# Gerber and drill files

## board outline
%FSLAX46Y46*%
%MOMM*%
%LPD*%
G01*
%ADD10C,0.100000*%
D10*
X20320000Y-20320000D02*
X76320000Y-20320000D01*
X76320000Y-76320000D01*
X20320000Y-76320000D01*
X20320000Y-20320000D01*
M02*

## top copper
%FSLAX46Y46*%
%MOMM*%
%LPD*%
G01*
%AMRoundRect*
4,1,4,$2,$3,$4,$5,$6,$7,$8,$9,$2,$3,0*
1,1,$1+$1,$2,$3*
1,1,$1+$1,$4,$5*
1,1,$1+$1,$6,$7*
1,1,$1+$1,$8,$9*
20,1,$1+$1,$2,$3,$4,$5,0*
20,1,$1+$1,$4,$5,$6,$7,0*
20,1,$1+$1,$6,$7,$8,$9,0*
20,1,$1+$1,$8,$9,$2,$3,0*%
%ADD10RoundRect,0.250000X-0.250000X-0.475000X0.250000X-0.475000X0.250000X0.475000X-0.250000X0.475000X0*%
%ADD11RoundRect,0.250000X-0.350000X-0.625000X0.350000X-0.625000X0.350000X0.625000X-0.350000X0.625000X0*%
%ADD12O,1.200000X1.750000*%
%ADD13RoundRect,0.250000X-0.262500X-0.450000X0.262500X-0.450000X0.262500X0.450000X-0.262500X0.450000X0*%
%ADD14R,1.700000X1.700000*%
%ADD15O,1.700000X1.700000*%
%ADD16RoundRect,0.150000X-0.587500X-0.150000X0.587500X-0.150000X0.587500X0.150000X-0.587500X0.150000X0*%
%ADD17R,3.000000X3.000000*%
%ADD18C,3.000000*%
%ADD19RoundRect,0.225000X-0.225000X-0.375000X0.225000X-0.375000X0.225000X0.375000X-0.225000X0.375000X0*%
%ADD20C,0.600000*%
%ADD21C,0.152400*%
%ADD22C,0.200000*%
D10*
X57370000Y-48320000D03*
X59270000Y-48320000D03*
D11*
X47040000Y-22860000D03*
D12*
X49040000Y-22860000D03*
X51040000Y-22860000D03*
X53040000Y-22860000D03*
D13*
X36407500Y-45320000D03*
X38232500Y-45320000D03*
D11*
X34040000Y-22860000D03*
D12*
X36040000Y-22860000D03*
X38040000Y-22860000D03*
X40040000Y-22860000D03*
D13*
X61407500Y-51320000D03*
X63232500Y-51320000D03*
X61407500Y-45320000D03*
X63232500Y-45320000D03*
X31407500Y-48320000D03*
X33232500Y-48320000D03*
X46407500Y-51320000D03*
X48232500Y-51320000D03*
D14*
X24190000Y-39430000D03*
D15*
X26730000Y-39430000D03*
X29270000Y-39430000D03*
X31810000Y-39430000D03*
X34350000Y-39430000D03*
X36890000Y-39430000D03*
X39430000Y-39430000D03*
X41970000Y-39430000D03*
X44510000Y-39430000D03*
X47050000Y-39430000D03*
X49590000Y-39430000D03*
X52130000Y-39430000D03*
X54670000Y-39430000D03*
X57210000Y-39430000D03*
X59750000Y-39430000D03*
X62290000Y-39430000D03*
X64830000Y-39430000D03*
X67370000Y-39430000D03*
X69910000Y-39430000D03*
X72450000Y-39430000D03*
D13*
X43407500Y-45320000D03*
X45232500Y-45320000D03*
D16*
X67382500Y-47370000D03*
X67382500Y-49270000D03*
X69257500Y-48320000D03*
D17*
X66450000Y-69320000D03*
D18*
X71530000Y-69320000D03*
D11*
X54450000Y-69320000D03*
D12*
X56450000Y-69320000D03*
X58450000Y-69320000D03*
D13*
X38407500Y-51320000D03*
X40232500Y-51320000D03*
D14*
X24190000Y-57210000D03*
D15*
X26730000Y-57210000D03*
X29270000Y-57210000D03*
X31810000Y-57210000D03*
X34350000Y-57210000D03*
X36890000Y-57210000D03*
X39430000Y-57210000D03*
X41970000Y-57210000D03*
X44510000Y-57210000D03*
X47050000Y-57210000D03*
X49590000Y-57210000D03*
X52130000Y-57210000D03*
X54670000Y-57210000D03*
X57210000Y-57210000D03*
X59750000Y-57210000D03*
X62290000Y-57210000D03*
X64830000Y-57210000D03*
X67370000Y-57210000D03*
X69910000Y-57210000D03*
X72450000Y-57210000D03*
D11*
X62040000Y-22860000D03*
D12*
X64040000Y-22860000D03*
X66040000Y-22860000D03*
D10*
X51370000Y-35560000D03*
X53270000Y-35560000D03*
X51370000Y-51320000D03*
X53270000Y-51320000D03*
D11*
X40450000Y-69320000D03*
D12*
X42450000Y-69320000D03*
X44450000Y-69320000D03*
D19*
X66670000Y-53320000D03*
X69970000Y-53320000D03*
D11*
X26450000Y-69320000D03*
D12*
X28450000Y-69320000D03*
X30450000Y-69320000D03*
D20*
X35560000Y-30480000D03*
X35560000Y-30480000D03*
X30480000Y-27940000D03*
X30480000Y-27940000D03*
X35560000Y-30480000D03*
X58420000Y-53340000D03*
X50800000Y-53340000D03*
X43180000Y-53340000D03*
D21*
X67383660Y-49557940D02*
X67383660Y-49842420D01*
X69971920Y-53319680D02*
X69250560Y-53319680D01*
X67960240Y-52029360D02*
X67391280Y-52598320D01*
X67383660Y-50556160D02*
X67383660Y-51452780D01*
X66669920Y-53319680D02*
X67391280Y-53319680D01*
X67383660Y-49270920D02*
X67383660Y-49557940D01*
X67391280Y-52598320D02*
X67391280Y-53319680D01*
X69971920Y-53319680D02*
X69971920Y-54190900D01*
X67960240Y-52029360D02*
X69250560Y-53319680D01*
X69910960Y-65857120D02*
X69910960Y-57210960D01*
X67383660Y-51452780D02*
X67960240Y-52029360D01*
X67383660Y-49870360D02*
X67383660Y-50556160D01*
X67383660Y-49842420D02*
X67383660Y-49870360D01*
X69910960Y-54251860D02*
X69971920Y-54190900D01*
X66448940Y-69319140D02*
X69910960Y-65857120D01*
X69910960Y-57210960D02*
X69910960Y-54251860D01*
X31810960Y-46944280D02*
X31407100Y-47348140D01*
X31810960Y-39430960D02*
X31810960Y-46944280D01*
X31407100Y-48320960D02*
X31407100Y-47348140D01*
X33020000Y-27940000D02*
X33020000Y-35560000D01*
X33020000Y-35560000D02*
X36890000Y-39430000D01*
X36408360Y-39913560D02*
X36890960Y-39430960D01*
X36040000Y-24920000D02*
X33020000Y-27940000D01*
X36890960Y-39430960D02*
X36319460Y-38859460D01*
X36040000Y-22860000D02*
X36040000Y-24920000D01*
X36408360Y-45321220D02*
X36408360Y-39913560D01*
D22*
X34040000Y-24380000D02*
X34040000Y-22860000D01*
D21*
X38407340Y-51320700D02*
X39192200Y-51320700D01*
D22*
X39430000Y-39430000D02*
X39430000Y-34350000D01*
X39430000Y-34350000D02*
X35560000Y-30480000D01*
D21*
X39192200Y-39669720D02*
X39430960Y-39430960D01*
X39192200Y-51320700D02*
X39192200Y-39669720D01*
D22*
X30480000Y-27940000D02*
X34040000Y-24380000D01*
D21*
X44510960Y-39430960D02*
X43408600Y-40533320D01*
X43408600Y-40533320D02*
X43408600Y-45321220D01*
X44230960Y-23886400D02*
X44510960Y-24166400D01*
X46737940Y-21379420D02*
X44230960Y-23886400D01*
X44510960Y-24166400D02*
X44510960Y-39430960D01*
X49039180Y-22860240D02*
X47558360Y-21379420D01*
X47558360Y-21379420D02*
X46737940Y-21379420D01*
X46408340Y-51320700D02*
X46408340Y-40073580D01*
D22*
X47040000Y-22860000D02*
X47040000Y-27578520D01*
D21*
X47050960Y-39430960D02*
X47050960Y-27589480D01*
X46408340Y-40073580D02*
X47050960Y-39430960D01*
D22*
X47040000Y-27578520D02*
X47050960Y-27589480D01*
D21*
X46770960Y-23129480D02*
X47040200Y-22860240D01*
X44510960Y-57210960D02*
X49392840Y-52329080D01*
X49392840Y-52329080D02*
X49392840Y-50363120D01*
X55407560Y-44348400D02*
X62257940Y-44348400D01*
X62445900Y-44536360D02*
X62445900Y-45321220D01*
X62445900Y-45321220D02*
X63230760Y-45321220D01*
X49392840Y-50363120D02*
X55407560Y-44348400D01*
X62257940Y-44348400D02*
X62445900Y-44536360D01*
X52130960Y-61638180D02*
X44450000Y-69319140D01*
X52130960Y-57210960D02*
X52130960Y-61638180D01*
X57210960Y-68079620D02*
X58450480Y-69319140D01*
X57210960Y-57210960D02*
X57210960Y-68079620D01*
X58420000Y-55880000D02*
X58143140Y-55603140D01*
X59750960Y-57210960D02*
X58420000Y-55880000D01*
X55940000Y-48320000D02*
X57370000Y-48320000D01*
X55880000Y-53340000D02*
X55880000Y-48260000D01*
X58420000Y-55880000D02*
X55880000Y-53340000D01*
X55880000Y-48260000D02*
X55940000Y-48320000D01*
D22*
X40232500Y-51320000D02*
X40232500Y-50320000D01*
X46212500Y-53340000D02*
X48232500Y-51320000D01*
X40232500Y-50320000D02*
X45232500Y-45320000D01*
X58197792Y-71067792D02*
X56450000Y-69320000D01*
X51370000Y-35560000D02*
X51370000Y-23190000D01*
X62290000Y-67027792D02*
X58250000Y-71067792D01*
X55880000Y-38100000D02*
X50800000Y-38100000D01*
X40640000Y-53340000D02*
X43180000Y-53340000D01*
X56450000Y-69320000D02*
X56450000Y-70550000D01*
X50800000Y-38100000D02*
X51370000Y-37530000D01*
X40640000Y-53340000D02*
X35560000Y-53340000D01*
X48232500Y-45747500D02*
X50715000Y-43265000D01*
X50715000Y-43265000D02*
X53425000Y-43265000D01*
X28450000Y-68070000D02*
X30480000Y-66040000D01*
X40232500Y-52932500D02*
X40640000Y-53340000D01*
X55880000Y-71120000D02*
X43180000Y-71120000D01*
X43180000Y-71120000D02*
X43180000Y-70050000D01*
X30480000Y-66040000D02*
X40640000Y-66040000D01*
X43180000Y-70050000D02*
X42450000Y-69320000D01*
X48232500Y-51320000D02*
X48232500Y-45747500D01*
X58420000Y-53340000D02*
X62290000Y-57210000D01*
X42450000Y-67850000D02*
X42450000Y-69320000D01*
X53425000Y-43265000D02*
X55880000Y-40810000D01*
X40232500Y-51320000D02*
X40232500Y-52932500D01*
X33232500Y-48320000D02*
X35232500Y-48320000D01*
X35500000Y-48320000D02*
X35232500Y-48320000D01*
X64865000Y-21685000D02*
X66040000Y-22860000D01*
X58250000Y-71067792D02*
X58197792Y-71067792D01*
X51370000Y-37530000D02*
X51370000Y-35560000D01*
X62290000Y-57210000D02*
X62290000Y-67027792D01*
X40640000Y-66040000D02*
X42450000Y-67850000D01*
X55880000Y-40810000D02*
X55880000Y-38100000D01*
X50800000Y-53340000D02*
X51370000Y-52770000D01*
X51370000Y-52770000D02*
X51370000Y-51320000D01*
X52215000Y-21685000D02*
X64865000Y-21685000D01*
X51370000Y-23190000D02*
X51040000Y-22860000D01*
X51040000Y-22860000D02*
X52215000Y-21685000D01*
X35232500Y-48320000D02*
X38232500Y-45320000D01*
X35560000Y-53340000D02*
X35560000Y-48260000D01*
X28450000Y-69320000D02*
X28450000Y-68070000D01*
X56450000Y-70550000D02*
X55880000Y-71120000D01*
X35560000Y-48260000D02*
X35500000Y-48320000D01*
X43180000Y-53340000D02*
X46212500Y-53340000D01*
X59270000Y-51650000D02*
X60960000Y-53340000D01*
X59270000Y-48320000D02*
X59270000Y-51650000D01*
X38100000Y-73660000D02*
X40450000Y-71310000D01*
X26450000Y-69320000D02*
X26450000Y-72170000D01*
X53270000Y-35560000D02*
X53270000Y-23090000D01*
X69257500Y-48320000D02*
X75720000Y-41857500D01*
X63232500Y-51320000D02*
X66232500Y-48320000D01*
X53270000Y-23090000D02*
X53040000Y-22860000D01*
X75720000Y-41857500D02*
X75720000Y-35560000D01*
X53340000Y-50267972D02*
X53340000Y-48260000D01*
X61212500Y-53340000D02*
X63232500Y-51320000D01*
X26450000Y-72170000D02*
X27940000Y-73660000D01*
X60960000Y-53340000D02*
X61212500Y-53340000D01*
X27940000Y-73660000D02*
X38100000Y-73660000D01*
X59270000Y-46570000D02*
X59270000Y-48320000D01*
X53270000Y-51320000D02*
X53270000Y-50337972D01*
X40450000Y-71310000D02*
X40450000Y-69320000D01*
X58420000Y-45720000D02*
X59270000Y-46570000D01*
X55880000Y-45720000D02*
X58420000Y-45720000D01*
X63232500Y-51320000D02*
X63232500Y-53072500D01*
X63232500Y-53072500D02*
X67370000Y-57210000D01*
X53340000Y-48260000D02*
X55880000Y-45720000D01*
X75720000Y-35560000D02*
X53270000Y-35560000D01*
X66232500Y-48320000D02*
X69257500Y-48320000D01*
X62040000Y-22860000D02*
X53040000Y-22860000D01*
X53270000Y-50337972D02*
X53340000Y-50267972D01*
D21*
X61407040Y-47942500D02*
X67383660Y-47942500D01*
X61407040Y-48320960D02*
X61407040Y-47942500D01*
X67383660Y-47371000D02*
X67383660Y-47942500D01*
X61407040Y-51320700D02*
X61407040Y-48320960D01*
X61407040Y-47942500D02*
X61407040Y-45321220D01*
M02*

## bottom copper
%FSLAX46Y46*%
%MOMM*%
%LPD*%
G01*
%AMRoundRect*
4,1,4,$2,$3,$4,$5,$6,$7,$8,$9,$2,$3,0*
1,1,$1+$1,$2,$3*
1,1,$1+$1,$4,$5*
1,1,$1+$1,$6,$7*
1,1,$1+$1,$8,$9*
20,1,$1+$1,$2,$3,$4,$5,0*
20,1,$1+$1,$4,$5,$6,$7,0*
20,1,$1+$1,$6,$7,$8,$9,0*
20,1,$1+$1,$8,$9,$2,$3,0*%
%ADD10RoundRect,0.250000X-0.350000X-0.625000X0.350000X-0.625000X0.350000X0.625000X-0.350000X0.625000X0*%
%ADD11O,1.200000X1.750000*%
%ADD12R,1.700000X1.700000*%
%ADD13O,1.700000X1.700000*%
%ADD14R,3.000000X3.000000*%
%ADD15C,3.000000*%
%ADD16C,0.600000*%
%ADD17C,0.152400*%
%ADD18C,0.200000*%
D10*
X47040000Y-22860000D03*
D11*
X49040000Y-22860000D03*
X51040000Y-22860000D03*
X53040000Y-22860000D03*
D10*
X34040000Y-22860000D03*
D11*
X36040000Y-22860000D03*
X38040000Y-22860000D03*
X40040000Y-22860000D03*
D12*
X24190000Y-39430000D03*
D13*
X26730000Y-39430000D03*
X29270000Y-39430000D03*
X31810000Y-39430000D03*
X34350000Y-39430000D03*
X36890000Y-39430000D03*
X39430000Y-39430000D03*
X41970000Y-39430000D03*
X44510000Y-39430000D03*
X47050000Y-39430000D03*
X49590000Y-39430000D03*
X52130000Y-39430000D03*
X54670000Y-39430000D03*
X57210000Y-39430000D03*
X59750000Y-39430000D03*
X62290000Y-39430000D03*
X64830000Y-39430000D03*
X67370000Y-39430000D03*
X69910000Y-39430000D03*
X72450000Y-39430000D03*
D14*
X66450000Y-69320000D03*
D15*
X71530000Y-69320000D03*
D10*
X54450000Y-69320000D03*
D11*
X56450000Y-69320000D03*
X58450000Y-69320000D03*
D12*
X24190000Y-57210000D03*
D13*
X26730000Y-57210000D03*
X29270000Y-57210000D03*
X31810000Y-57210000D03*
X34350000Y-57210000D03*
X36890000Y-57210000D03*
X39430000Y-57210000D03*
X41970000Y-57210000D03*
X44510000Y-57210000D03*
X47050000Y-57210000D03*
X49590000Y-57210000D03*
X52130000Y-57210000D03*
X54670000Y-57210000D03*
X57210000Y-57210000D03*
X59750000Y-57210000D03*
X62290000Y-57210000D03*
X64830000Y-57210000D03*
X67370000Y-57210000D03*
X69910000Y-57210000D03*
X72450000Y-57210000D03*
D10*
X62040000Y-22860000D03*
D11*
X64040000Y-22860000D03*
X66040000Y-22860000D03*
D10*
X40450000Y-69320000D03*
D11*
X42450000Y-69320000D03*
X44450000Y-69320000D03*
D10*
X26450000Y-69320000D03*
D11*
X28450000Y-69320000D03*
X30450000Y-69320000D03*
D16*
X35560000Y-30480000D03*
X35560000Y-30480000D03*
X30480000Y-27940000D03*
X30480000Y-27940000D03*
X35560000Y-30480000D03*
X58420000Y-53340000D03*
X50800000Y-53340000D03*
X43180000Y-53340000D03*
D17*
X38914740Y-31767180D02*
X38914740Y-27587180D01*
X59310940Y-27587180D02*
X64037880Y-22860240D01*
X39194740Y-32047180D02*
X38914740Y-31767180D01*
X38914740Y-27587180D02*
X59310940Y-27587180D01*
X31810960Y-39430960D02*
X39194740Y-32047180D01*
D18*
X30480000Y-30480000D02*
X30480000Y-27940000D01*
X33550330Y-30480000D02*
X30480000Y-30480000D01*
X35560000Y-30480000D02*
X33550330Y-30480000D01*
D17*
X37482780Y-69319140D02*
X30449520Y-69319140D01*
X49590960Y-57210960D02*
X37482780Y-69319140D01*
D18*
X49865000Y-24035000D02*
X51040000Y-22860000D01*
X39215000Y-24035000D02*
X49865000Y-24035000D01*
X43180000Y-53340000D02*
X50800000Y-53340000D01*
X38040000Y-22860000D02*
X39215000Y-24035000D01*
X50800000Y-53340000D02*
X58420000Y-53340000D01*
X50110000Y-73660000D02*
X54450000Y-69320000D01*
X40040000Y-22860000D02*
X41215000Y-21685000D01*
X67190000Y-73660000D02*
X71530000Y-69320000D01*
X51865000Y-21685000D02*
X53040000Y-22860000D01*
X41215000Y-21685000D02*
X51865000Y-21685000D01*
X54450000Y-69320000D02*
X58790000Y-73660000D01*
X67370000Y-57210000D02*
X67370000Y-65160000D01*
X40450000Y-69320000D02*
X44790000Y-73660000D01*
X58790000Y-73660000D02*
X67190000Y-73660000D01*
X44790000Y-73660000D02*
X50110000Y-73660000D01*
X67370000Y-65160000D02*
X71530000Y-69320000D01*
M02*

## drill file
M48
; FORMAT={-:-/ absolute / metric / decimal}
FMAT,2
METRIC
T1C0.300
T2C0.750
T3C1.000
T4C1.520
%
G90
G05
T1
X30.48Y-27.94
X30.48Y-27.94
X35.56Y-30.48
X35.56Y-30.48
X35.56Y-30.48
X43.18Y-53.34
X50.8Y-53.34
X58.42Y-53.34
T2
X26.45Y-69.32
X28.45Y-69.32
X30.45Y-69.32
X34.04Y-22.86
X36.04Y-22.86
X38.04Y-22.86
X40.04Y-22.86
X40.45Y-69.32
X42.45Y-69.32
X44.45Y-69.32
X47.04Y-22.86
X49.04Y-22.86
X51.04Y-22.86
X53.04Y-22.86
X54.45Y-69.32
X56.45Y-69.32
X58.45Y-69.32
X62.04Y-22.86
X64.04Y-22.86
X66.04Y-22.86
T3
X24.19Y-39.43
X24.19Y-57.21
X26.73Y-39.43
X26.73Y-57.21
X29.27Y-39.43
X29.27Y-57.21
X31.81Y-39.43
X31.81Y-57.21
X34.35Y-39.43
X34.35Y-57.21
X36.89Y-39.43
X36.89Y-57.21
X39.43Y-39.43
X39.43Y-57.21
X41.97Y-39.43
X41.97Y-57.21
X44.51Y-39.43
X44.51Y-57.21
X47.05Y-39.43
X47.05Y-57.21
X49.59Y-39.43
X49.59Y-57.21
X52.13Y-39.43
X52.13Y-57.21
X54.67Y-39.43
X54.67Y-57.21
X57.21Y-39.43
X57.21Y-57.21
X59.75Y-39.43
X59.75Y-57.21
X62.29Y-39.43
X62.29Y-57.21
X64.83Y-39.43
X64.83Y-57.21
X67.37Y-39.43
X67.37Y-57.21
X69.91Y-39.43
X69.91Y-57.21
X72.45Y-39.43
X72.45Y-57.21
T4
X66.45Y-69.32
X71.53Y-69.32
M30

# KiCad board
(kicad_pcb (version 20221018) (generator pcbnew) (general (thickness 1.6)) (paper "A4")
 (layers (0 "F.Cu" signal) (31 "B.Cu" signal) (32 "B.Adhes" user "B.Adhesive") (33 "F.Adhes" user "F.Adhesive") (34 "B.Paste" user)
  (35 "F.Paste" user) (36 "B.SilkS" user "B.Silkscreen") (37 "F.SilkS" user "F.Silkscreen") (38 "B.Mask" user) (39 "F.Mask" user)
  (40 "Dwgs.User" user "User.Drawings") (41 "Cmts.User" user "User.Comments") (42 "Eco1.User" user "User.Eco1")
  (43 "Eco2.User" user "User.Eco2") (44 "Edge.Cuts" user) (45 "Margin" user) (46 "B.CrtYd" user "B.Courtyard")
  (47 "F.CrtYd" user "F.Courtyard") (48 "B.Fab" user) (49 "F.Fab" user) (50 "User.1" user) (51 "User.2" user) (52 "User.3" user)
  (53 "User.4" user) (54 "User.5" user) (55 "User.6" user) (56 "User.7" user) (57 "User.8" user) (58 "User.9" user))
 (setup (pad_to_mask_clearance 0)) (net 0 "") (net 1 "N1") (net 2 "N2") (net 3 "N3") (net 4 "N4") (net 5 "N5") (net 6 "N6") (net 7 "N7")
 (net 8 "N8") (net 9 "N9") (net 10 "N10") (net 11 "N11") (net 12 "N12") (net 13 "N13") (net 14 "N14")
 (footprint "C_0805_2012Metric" (layer "F.Cu") (at 58.32 48.32)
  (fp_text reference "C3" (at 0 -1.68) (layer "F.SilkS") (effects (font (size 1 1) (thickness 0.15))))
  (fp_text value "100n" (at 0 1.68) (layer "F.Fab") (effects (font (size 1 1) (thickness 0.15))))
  (pad "1" smd roundrect (at -0.95 0) (size 1 1.45) (layers "F.Cu" "F.Paste" "F.Mask") (roundrect_rratio 0.25) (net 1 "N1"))
  (pad "2" smd roundrect (at 0.95 0) (size 1 1.45) (layers "F.Cu" "F.Paste" "F.Mask") (roundrect_rratio 0.25) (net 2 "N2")))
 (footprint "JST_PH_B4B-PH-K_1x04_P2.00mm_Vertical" (layer "F.Cu") (at 47.04 22.86)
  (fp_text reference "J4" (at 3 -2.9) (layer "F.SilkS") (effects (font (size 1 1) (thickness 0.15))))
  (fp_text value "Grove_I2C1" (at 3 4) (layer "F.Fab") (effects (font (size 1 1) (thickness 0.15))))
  (pad "1" thru_hole roundrect (at 0 0) (size 1.2 1.75) (drill 0.75) (layers "*.Cu" "*.Mask") (roundrect_rratio 0.208333) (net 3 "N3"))
  (pad "2" thru_hole oval (at 2 0) (size 1.2 1.75) (drill 0.75) (layers "*.Cu" "*.Mask") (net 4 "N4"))
  (pad "3" thru_hole oval (at 4 0) (size 1.2 1.75) (drill 0.75) (layers "*.Cu" "*.Mask") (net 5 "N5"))
  (pad "4" thru_hole oval (at 6 0) (size 1.2 1.75) (drill 0.75) (layers "*.Cu" "*.Mask") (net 2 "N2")))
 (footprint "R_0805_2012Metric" (layer "F.Cu") (at 37.32 45.32)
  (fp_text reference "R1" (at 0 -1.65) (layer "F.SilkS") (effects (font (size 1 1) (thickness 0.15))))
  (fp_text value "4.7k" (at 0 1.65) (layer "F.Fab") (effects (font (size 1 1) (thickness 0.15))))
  (pad "1" smd roundrect (at -0.9125 0) (size 1.025 1.4) (layers "F.Cu" "F.Paste" "F.Mask") (roundrect_rratio 0.243902) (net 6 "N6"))
  (pad "2" smd roundrect (at 0.9125 0) (size 1.025 1.4) (layers "F.Cu" "F.Paste" "F.Mask") (roundrect_rratio 0.243902) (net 5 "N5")))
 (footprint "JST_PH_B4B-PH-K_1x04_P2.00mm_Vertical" (layer "F.Cu") (at 34.04 22.86)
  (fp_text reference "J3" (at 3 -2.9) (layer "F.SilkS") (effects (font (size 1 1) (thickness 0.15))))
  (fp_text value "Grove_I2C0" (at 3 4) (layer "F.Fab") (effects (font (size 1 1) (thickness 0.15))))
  (pad "1" thru_hole roundrect (at 0 0) (size 1.2 1.75) (drill 0.75) (layers "*.Cu" "*.Mask") (roundrect_rratio 0.208333) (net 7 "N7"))
  (pad "2" thru_hole oval (at 2 0) (size 1.2 1.75) (drill 0.75) (layers "*.Cu" "*.Mask") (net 6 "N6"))
  (pad "3" thru_hole oval (at 4 0) (size 1.2 1.75) (drill 0.75) (layers "*.Cu" "*.Mask") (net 5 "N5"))
  (pad "4" thru_hole oval (at 6 0) (size 1.2 1.75) (drill 0.75) (layers "*.Cu" "*.Mask") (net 2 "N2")))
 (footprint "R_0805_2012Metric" (layer "F.Cu") (at 62.32 51.32)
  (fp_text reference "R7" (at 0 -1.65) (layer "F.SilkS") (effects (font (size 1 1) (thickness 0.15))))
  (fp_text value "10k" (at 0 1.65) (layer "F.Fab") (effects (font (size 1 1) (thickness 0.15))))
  (pad "1" smd roundrect (at -0.9125 0) (size 1.025 1.4) (layers "F.Cu" "F.Paste" "F.Mask") (roundrect_rratio 0.243902) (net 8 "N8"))
  (pad "2" smd roundrect (at 0.9125 0) (size 1.025 1.4) (layers "F.Cu" "F.Paste" "F.Mask") (roundrect_rratio 0.243902) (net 2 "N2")))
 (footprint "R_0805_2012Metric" (layer "F.Cu") (at 62.32 45.32)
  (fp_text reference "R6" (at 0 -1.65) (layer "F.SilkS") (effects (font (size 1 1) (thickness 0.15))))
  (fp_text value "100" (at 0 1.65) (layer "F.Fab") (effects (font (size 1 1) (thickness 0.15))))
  (pad "1" smd roundrect (at -0.9125 0) (size 1.025 1.4) (layers "F.Cu" "F.Paste" "F.Mask") (roundrect_rratio 0.243902) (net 8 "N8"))
  (pad "2" smd roundrect (at 0.9125 0) (size 1.025 1.4) (layers "F.Cu" "F.Paste" "F.Mask") (roundrect_rratio 0.243902) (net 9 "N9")))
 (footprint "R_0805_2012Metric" (layer "F.Cu") (at 32.32 48.32)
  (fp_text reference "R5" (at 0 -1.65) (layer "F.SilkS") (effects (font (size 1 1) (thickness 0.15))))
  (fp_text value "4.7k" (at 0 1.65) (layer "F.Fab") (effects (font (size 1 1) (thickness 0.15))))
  (pad "1" smd roundrect (at -0.9125 0) (size 1.025 1.4) (layers "F.Cu" "F.Paste" "F.Mask") (roundrect_rratio 0.243902) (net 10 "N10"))
  (pad "2" smd roundrect (at 0.9125 0) (size 1.025 1.4) (layers "F.Cu" "F.Paste" "F.Mask") (roundrect_rratio 0.243902) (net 5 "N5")))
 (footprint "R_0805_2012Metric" (layer "F.Cu") (at 47.32 51.32)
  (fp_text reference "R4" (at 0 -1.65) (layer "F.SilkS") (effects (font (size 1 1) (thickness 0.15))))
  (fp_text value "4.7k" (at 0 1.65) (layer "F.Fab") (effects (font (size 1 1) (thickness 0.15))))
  (pad "1" smd roundrect (at -0.9125 0) (size 1.025 1.4) (layers "F.Cu" "F.Paste" "F.Mask") (roundrect_rratio 0.243902) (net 3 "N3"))
  (pad "2" smd roundrect (at 0.9125 0) (size 1.025 1.4) (layers "F.Cu" "F.Paste" "F.Mask") (roundrect_rratio 0.243902) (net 5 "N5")))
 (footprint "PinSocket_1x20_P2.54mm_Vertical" (layer "F.Cu") (at 24.19 39.43 90)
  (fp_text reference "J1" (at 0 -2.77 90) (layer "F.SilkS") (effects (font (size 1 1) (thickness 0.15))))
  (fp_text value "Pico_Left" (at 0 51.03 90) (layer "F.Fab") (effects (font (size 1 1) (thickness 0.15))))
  (pad "1" thru_hole rect (at 0 0 90) (size 1.7 1.7) (drill 1) (layers "*.Cu" "*.Mask"))
  (pad "2" thru_hole oval (at 0 2.54 90) (size 1.7 1.7) (drill 1) (layers "*.Cu" "*.Mask"))
  (pad "3" thru_hole oval (at 0 5.08 90) (size 1.7 1.7) (drill 1) (layers "*.Cu" "*.Mask"))
  (pad "4" thru_hole oval (at 0 7.62 90) (size 1.7 1.7) (drill 1) (layers "*.Cu" "*.Mask") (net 10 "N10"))
  (pad "5" thru_hole oval (at 0 10.16 90) (size 1.7 1.7) (drill 1) (layers "*.Cu" "*.Mask"))
  (pad "6" thru_hole oval (at 0 12.7 90) (size 1.7 1.7) (drill 1) (layers "*.Cu" "*.Mask") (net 6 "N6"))
  (pad "7" thru_hole oval (at 0 15.24 90) (size 1.7 1.7) (drill 1) (layers "*.Cu" "*.Mask") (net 7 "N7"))
  (pad "8" thru_hole oval (at 0 17.78 90) (size 1.7 1.7) (drill 1) (layers "*.Cu" "*.Mask"))
  (pad "9" thru_hole oval (at 0 20.32 90) (size 1.7 1.7) (drill 1) (layers "*.Cu" "*.Mask") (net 4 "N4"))
  (pad "10" thru_hole oval (at 0 22.86 90) (size 1.7 1.7) (drill 1) (layers "*.Cu" "*.Mask") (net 3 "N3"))
  (pad "11" thru_hole oval (at 0 25.4 90) (size 1.7 1.7) (drill 1) (layers "*.Cu" "*.Mask"))
  (pad "12" thru_hole oval (at 0 27.94 90) (size 1.7 1.7) (drill 1) (layers "*.Cu" "*.Mask"))
  (pad "13" thru_hole oval (at 0 30.48 90) (size 1.7 1.7) (drill 1) (layers "*.Cu" "*.Mask"))
  (pad "14" thru_hole oval (at 0 33.02 90) (size 1.7 1.7) (drill 1) (layers "*.Cu" "*.Mask"))
  (pad "15" thru_hole oval (at 0 35.56 90) (size 1.7 1.7) (drill 1) (layers "*.Cu" "*.Mask"))
  (pad "16" thru_hole oval (at 0 38.1 90) (size 1.7 1.7) (drill 1) (layers "*.Cu" "*.Mask"))
  (pad "17" thru_hole oval (at 0 40.64 90) (size 1.7 1.7) (drill 1) (layers "*.Cu" "*.Mask"))
  (pad "18" thru_hole oval (at 0 43.18 90) (size 1.7 1.7) (drill 1) (layers "*.Cu" "*.Mask"))
  (pad "19" thru_hole oval (at 0 45.72 90) (size 1.7 1.7) (drill 1) (layers "*.Cu" "*.Mask"))
  (pad "20" thru_hole oval (at 0 48.26 90) (size 1.7 1.7) (drill 1) (layers "*.Cu" "*.Mask")))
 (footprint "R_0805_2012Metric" (layer "F.Cu") (at 44.32 45.32)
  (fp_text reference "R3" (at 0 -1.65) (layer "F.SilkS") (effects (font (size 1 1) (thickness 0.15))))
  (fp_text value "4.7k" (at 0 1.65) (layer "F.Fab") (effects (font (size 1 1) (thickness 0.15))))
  (pad "1" smd roundrect (at -0.9125 0) (size 1.025 1.4) (layers "F.Cu" "F.Paste" "F.Mask") (roundrect_rratio 0.243902) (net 4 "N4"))
  (pad "2" smd roundrect (at 0.9125 0) (size 1.025 1.4) (layers "F.Cu" "F.Paste" "F.Mask") (roundrect_rratio 0.243902) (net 5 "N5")))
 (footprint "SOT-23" (layer "F.Cu") (at 68.32 48.32)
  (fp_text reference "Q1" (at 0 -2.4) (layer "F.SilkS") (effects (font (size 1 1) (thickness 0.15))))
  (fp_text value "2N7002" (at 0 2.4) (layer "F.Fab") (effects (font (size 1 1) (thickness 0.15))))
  (pad "1" smd roundrect (at -0.9375 -0.95) (size 1.475 0.6) (layers "F.Cu" "F.Paste" "F.Mask") (roundrect_rratio 0.25) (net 8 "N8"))
  (pad "2" smd roundrect (at -0.9375 0.95) (size 1.475 0.6) (layers "F.Cu" "F.Paste" "F.Mask") (roundrect_rratio 0.25) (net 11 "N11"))
  (pad "3" smd roundrect (at 0.9375 0) (size 1.475 0.6) (layers "F.Cu" "F.Paste" "F.Mask") (roundrect_rratio 0.25) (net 2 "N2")))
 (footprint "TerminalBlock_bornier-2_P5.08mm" (layer "F.Cu") (at 66.45 69.32)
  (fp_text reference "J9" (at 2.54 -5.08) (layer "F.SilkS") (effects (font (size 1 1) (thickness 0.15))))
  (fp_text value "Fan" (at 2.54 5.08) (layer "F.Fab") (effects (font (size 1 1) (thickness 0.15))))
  (pad "1" thru_hole rect (at 0 0) (size 3 3) (drill 1.52) (layers "*.Cu" "*.Mask") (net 11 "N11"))
  (pad "2" thru_hole circle (at 5.08 0) (size 3 3) (drill 1.52) (layers "*.Cu" "*.Mask") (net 2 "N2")))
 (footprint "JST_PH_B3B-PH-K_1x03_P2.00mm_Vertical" (layer "F.Cu") (at 54.45 69.32)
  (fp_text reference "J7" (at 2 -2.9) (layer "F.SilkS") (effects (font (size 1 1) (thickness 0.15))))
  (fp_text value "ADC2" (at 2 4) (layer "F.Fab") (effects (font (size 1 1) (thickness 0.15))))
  (pad "1" thru_hole roundrect (at 0 0) (size 1.2 1.75) (drill 0.75) (layers "*.Cu" "*.Mask") (roundrect_rratio 0.208333) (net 2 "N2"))
  (pad "2" thru_hole oval (at 2 0) (size 1.2 1.75) (drill 0.75) (layers "*.Cu" "*.Mask") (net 5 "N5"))
  (pad "3" thru_hole oval (at 4 0) (size 1.2 1.75) (drill 0.75) (layers "*.Cu" "*.Mask") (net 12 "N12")))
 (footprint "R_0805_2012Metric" (layer "F.Cu") (at 39.32 51.32)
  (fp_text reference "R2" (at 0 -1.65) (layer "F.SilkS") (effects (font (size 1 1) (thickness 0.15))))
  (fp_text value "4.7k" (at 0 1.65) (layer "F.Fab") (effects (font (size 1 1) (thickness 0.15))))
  (pad "1" smd roundrect (at -0.9125 0) (size 1.025 1.4) (layers "F.Cu" "F.Paste" "F.Mask") (roundrect_rratio 0.243902) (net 7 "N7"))
  (pad "2" smd roundrect (at 0.9125 0) (size 1.025 1.4) (layers "F.Cu" "F.Paste" "F.Mask") (roundrect_rratio 0.243902) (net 5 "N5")))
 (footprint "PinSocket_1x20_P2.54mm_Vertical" (layer "F.Cu") (at 24.19 57.21 90)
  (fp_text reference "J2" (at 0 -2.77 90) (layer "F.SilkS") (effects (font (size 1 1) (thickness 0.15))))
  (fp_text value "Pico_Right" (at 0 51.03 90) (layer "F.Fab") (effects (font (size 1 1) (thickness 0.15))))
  (pad "1" thru_hole rect (at 0 0 90) (size 1.7 1.7) (drill 1) (layers "*.Cu" "*.Mask"))
  (pad "2" thru_hole oval (at 0 2.54 90) (size 1.7 1.7) (drill 1) (layers "*.Cu" "*.Mask"))
  (pad "3" thru_hole oval (at 0 5.08 90) (size 1.7 1.7) (drill 1) (layers "*.Cu" "*.Mask"))
  (pad "4" thru_hole oval (at 0 7.62 90) (size 1.7 1.7) (drill 1) (layers "*.Cu" "*.Mask"))
  (pad "5" thru_hole oval (at 0 10.16 90) (size 1.7 1.7) (drill 1) (layers "*.Cu" "*.Mask"))
  (pad "6" thru_hole oval (at 0 12.7 90) (size 1.7 1.7) (drill 1) (layers "*.Cu" "*.Mask"))
  (pad "7" thru_hole oval (at 0 15.24 90) (size 1.7 1.7) (drill 1) (layers "*.Cu" "*.Mask"))
  (pad "8" thru_hole oval (at 0 17.78 90) (size 1.7 1.7) (drill 1) (layers "*.Cu" "*.Mask"))
  (pad "9" thru_hole oval (at 0 20.32 90) (size 1.7 1.7) (drill 1) (layers "*.Cu" "*.Mask") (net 9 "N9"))
  (pad "10" thru_hole oval (at 0 22.86 90) (size 1.7 1.7) (drill 1) (layers "*.Cu" "*.Mask"))
  (pad "11" thru_hole oval (at 0 25.4 90) (size 1.7 1.7) (drill 1) (layers "*.Cu" "*.Mask") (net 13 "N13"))
  (pad "12" thru_hole oval (at 0 27.94 90) (size 1.7 1.7) (drill 1) (layers "*.Cu" "*.Mask") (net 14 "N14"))
  (pad "13" thru_hole oval (at 0 30.48 90) (size 1.7 1.7) (drill 1) (layers "*.Cu" "*.Mask"))
  (pad "14" thru_hole oval (at 0 33.02 90) (size 1.7 1.7) (drill 1) (layers "*.Cu" "*.Mask") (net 12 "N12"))
  (pad "15" thru_hole oval (at 0 35.56 90) (size 1.7 1.7) (drill 1) (layers "*.Cu" "*.Mask") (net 1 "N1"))
  (pad "16" thru_hole oval (at 0 38.1 90) (size 1.7 1.7) (drill 1) (layers "*.Cu" "*.Mask") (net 5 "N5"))
  (pad "17" thru_hole oval (at 0 40.64 90) (size 1.7 1.7) (drill 1) (layers "*.Cu" "*.Mask"))
  (pad "18" thru_hole oval (at 0 43.18 90) (size 1.7 1.7) (drill 1) (layers "*.Cu" "*.Mask") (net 2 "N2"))
  (pad "19" thru_hole oval (at 0 45.72 90) (size 1.7 1.7) (drill 1) (layers "*.Cu" "*.Mask") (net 11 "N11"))
  (pad "20" thru_hole oval (at 0 48.26 90) (size 1.7 1.7) (drill 1) (layers "*.Cu" "*.Mask")))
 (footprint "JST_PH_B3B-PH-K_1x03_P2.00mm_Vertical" (layer "F.Cu") (at 62.04 22.86)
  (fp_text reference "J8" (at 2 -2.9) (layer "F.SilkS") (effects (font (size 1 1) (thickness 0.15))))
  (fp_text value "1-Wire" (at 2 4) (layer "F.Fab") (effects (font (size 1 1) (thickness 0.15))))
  (pad "1" thru_hole roundrect (at 0 0) (size 1.2 1.75) (drill 0.75) (layers "*.Cu" "*.Mask") (roundrect_rratio 0.208333) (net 2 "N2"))
  (pad "2" thru_hole oval (at 2 0) (size 1.2 1.75) (drill 0.75) (layers "*.Cu" "*.Mask") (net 10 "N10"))
  (pad "3" thru_hole oval (at 4 0) (size 1.2 1.75) (drill 0.75) (layers "*.Cu" "*.Mask") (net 5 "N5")))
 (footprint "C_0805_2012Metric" (layer "F.Cu") (at 52.32 35.56)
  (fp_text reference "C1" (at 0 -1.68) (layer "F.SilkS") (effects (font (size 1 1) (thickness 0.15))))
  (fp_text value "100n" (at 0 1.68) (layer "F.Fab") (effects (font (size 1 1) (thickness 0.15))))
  (pad "1" smd roundrect (at -0.95 0) (size 1 1.45) (layers "F.Cu" "F.Paste" "F.Mask") (roundrect_rratio 0.25) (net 5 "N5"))
  (pad "2" smd roundrect (at 0.95 0) (size 1 1.45) (layers "F.Cu" "F.Paste" "F.Mask") (roundrect_rratio 0.25) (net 2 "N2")))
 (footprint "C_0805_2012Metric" (layer "F.Cu") (at 52.32 51.32)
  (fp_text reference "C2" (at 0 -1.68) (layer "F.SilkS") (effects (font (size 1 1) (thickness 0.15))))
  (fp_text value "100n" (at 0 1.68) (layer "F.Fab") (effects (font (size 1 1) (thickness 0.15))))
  (pad "1" smd roundrect (at -0.95 0) (size 1 1.45) (layers "F.Cu" "F.Paste" "F.Mask") (roundrect_rratio 0.25) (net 5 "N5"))
  (pad "2" smd roundrect (at 0.95 0) (size 1 1.45) (layers "F.Cu" "F.Paste" "F.Mask") (roundrect_rratio 0.25) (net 2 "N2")))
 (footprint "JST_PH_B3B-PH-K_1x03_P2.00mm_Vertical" (layer "F.Cu") (at 40.45 69.32)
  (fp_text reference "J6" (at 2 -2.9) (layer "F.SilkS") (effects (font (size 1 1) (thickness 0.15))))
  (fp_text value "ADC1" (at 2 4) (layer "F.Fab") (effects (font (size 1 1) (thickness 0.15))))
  (pad "1" thru_hole roundrect (at 0 0) (size 1.2 1.75) (drill 0.75) (layers "*.Cu" "*.Mask") (roundrect_rratio 0.208333) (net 2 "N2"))
  (pad "2" thru_hole oval (at 2 0) (size 1.2 1.75) (drill 0.75) (layers "*.Cu" "*.Mask") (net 5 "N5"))
  (pad "3" thru_hole oval (at 4 0) (size 1.2 1.75) (drill 0.75) (layers "*.Cu" "*.Mask") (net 14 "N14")))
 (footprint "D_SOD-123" (layer "F.Cu") (at 68.32 53.32)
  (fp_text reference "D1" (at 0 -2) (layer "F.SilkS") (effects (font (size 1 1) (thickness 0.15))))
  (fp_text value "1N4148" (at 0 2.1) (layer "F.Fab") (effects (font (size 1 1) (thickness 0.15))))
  (pad "1" smd roundrect (at -1.65 0) (size 0.9 1.2) (layers "F.Cu" "F.Paste" "F.Mask") (roundrect_rratio 0.25) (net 11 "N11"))
  (pad "2" smd roundrect (at 1.65 0) (size 0.9 1.2) (layers "F.Cu" "F.Paste" "F.Mask") (roundrect_rratio 0.25) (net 11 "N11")))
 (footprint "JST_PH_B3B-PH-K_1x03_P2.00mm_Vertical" (layer "F.Cu") (at 26.45 69.32)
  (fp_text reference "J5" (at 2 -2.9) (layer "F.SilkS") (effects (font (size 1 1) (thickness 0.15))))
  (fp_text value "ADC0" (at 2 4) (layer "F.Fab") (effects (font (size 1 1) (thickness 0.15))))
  (pad "1" thru_hole roundrect (at 0 0) (size 1.2 1.75) (drill 0.75) (layers "*.Cu" "*.Mask") (roundrect_rratio 0.208333) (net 2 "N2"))
  (pad "2" thru_hole oval (at 2 0) (size 1.2 1.75) (drill 0.75) (layers "*.Cu" "*.Mask") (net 5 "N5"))
  (pad "3" thru_hole oval (at 4 0) (size 1.2 1.75) (drill 0.75) (layers "*.Cu" "*.Mask") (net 13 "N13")))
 (gr_rect (start 20.32 20.32) (end 76.32 76.32) (stroke (width 0.1) (type default)) (fill none) (layer "Edge.Cuts"))
 (segment (start 67.38366 49.55794) (end 67.38366 49.84242) (width 0.1524) (layer "F.Cu") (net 11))
 (segment (start 69.97192 53.31968) (end 69.25056 53.31968) (width 0.1524) (layer "F.Cu") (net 11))
 (segment (start 67.96024 52.02936) (end 67.39128 52.59832) (width 0.1524) (layer "F.Cu") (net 11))
 (segment (start 67.38366 50.55616) (end 67.38366 51.45278) (width 0.1524) (layer "F.Cu") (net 11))
 (segment (start 66.66992 53.31968) (end 67.39128 53.31968) (width 0.1524) (layer "F.Cu") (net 11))
 (segment (start 67.38366 49.27092) (end 67.38366 49.55794) (width 0.1524) (layer "F.Cu") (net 11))
 (segment (start 67.39128 52.59832) (end 67.39128 53.31968) (width 0.1524) (layer "F.Cu") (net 11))
 (segment (start 69.97192 53.31968) (end 69.97192 54.1909) (width 0.1524) (layer "F.Cu") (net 11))
 (segment (start 67.96024 52.02936) (end 69.25056 53.31968) (width 0.1524) (layer "F.Cu") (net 11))
 (segment (start 69.91096 65.85712) (end 69.91096 57.21096) (width 0.1524) (layer "F.Cu") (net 11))
 (segment (start 67.38366 51.45278) (end 67.96024 52.02936) (width 0.1524) (layer "F.Cu") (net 11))
 (segment (start 67.38366 49.87036) (end 67.38366 50.55616) (width 0.1524) (layer "F.Cu") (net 11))
 (segment (start 67.38366 49.84242) (end 67.38366 49.87036) (width 0.1524) (layer "F.Cu") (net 11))
 (segment (start 69.91096 54.25186) (end 69.97192 54.1909) (width 0.1524) (layer "F.Cu") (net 11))
 (segment (start 66.44894 69.31914) (end 69.91096 65.85712) (width 0.1524) (layer "F.Cu") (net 11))
 (segment (start 69.91096 57.21096) (end 69.91096 54.25186) (width 0.1524) (layer "F.Cu") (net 11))
 (segment (start 31.81096 46.94428) (end 31.4071 47.34814) (width 0.1524) (layer "F.Cu") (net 10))
 (segment (start 31.81096 39.43096) (end 31.81096 46.94428) (width 0.1524) (layer "F.Cu") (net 10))
 (segment (start 31.4071 48.32096) (end 31.4071 47.34814) (width 0.1524) (layer "F.Cu") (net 10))
 (segment (start 38.91474 31.76718) (end 38.91474 27.58718) (width 0.1524) (layer "B.Cu") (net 10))
 (segment (start 59.31094 27.58718) (end 64.03788 22.86024) (width 0.1524) (layer "B.Cu") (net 10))
 (segment (start 39.19474 32.04718) (end 38.91474 31.76718) (width 0.1524) (layer "B.Cu") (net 10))
 (segment (start 38.91474 27.58718) (end 59.31094 27.58718) (width 0.1524) (layer "B.Cu") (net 10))
 (segment (start 31.81096 39.43096) (end 39.19474 32.04718) (width 0.1524) (layer "B.Cu") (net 10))
 (segment (start 33.02 27.94) (end 33.02 35.56) (width 0.1524) (layer "F.Cu") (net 6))
 (segment (start 33.02 35.56) (end 36.89 39.43) (width 0.1524) (layer "F.Cu") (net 6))
 (segment (start 36.40836 39.91356) (end 36.89096 39.43096) (width 0.1524) (layer "F.Cu") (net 6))
 (segment (start 36.04 24.92) (end 33.02 27.94) (width 0.1524) (layer "F.Cu") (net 6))
 (segment (start 36.89096 39.43096) (end 36.31946 38.85946) (width 0.1524) (layer "F.Cu") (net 6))
 (segment (start 36.04 22.86) (end 36.04 24.92) (width 0.1524) (layer "F.Cu") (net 6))
 (segment (start 36.40836 45.32122) (end 36.40836 39.91356) (width 0.1524) (layer "F.Cu") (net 6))
 (segment (start 34.04 24.38) (end 34.04 22.86) (width 0.2) (layer "F.Cu") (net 7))
 (segment (start 38.40734 51.3207) (end 39.1922 51.3207) (width 0.1524) (layer "F.Cu") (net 7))
 (segment (start 39.43 39.43) (end 39.43 34.35) (width 0.2) (layer "F.Cu") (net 7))
 (segment (start 39.43 34.35) (end 35.56 30.48) (width 0.2) (layer "F.Cu") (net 7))
 (segment (start 39.1922 39.66972) (end 39.43096 39.43096) (width 0.1524) (layer "F.Cu") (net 7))
 (segment (start 39.1922 51.3207) (end 39.1922 39.66972) (width 0.1524) (layer "F.Cu") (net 7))
 (segment (start 30.48 27.94) (end 34.04 24.38) (width 0.2) (layer "F.Cu") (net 7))
 (via (at 35.56 30.48) (size 0.6) (drill 0.3) (layers "F.Cu" "B.Cu") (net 7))
 (via (at 35.56 30.48) (size 0.6) (drill 0.3) (layers "F.Cu" "B.Cu") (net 7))
 (via (at 30.48 27.94) (size 0.6) (drill 0.3) (layers "F.Cu" "B.Cu") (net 7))
 (via (at 30.48 27.94) (size 0.6) (drill 0.3) (layers "F.Cu" "B.Cu") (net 7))
 (via (at 35.56 30.48) (size 0.6) (drill 0.3) (layers "F.Cu" "B.Cu") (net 7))
 (segment (start 30.48 30.48) (end 30.48 27.94) (width 0.2) (layer "B.Cu") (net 7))
 (segment (start 33.55033 30.48) (end 30.48 30.48) (width 0.2) (layer "B.Cu") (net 7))
 (segment (start 35.56 30.48) (end 33.55033 30.48) (width 0.2) (layer "B.Cu") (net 7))
 (segment (start 44.51096 39.43096) (end 43.4086 40.53332) (width 0.1524) (layer "F.Cu") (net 4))
 (segment (start 43.4086 40.53332) (end 43.4086 45.32122) (width 0.1524) (layer "F.Cu") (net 4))
 (segment (start 44.23096 23.8864) (end 44.51096 24.1664) (width 0.1524) (layer "F.Cu") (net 4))
 (segment (start 46.73794 21.37942) (end 44.23096 23.8864) (width 0.1524) (layer "F.Cu") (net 4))
 (segment (start 44.51096 24.1664) (end 44.51096 39.43096) (width 0.1524) (layer "F.Cu") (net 4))
 (segment (start 49.03918 22.86024) (end 47.55836 21.37942) (width 0.1524) (layer "F.Cu") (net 4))
 (segment (start 47.55836 21.37942) (end 46.73794 21.37942) (width 0.1524) (layer "F.Cu") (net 4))
 (segment (start 46.40834 51.3207) (end 46.40834 40.07358) (width 0.1524) (layer "F.Cu") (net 3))
 (segment (start 47.04 22.86) (end 47.04 27.57852) (width 0.2) (layer "F.Cu") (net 3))
 (segment (start 47.05096 39.43096) (end 47.05096 27.58948) (width 0.1524) (layer "F.Cu") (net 3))
 (segment (start 46.40834 40.07358) (end 47.05096 39.43096) (width 0.1524) (layer "F.Cu") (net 3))
 (segment (start 47.04 27.57852) (end 47.05096 27.58948) (width 0.2) (layer "F.Cu") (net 3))
 (segment (start 46.77096 23.12948) (end 47.0402 22.86024) (width 0.1524) (layer "F.Cu") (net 3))
 (segment (start 44.51096 57.21096) (end 49.39284 52.32908) (width 0.1524) (layer "F.Cu") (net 9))
 (segment (start 49.39284 52.32908) (end 49.39284 50.36312) (width 0.1524) (layer "F.Cu") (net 9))
 (segment (start 55.40756 44.3484) (end 62.25794 44.3484) (width 0.1524) (layer "F.Cu") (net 9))
 (segment (start 62.4459 44.53636) (end 62.4459 45.32122) (width 0.1524) (layer "F.Cu") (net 9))
 (segment (start 62.4459 45.32122) (end 63.23076 45.32122) (width 0.1524) (layer "F.Cu") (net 9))
 (segment (start 49.39284 50.36312) (end 55.40756 44.3484) (width 0.1524) (layer "F.Cu") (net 9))
 (segment (start 62.25794 44.3484) (end 62.4459 44.53636) (width 0.1524) (layer "F.Cu") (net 9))
 (segment (start 37.48278 69.31914) (end 30.44952 69.31914) (width 0.1524) (layer "B.Cu") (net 13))
 (segment (start 49.59096 57.21096) (end 37.48278 69.31914) (width 0.1524) (layer "B.Cu") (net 13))
 (segment (start 52.13096 61.63818) (end 44.45 69.31914) (width 0.1524) (layer "F.Cu") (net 14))
 (segment (start 52.13096 57.21096) (end 52.13096 61.63818) (width 0.1524) (layer "F.Cu") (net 14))
 (segment (start 57.21096 68.07962) (end 58.45048 69.31914) (width 0.1524) (layer "F.Cu") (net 12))
 (segment (start 57.21096 57.21096) (end 57.21096 68.07962) (width 0.1524) (layer "F.Cu") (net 12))
 (segment (start 58.42 55.88) (end 58.14314 55.60314) (width 0.1524) (layer "F.Cu") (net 1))
 (segment (start 59.75096 57.21096) (end 58.42 55.88) (width 0.1524) (layer "F.Cu") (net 1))
 (segment (start 55.94 48.32) (end 57.37 48.32) (width 0.1524) (layer "F.Cu") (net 1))
 (segment (start 55.88 53.34) (end 55.88 48.26) (width 0.1524) (layer "F.Cu") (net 1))
 (segment (start 58.42 55.88) (end 55.88 53.34) (width 0.1524) (layer "F.Cu") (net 1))
 (segment (start 55.88 48.26) (end 55.94 48.32) (width 0.1524) (layer "F.Cu") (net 1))
 (segment (start 40.2325 51.32) (end 40.2325 50.32) (width 0.2) (layer "F.Cu") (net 5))
 (segment (start 46.2125 53.34) (end 48.2325 51.32) (width 0.2) (layer "F.Cu") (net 5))
 (segment (start 40.2325 50.32) (end 45.2325 45.32) (width 0.2) (layer "F.Cu") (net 5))
 (segment (start 58.197792 71.067792) (end 56.45 69.32) (width 0.2) (layer "F.Cu") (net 5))
 (segment (start 51.37 35.56) (end 51.37 23.19) (width 0.2) (layer "F.Cu") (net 5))
 (segment (start 62.29 67.027792) (end 58.25 71.067792) (width 0.2) (layer "F.Cu") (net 5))
 (segment (start 55.88 38.1) (end 50.8 38.1) (width 0.2) (layer "F.Cu") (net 5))
 (segment (start 40.64 53.34) (end 43.18 53.34) (width 0.2) (layer "F.Cu") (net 5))
 (segment (start 56.45 69.32) (end 56.45 70.55) (width 0.2) (layer "F.Cu") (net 5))
 (segment (start 50.8 38.1) (end 51.37 37.53) (width 0.2) (layer "F.Cu") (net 5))
 (segment (start 40.64 53.34) (end 35.56 53.34) (width 0.2) (layer "F.Cu") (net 5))
 (segment (start 48.2325 45.7475) (end 50.715 43.265) (width 0.2) (layer "F.Cu") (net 5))
 (segment (start 50.715 43.265) (end 53.425 43.265) (width 0.2) (layer "F.Cu") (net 5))
 (segment (start 28.45 68.07) (end 30.48 66.04) (width 0.2) (layer "F.Cu") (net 5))
 (segment (start 40.2325 52.9325) (end 40.64 53.34) (width 0.2) (layer "F.Cu") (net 5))
 (segment (start 55.88 71.12) (end 43.18 71.12) (width 0.2) (layer "F.Cu") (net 5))
 (segment (start 43.18 71.12) (end 43.18 70.05) (width 0.2) (layer "F.Cu") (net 5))
 (segment (start 30.48 66.04) (end 40.64 66.04) (width 0.2) (layer "F.Cu") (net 5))
 (segment (start 43.18 70.05) (end 42.45 69.32) (width 0.2) (layer "F.Cu") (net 5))
 (segment (start 48.2325 51.32) (end 48.2325 45.7475) (width 0.2) (layer "F.Cu") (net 5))
 (segment (start 58.42 53.34) (end 62.29 57.21) (width 0.2) (layer "F.Cu") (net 5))
 (segment (start 42.45 67.85) (end 42.45 69.32) (width 0.2) (layer "F.Cu") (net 5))
 (segment (start 53.425 43.265) (end 55.88 40.81) (width 0.2) (layer "F.Cu") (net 5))
 (segment (start 40.2325 51.32) (end 40.2325 52.9325) (width 0.2) (layer "F.Cu") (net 5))
 (segment (start 33.2325 48.32) (end 35.2325 48.32) (width 0.2) (layer "F.Cu") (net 5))
 (segment (start 35.5 48.32) (end 35.2325 48.32) (width 0.2) (layer "F.Cu") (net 5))
 (segment (start 64.865 21.685) (end 66.04 22.86) (width 0.2) (layer "F.Cu") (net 5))
 (segment (start 58.25 71.067792) (end 58.197792 71.067792) (width 0.2) (layer "F.Cu") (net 5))
 (segment (start 51.37 37.53) (end 51.37 35.56) (width 0.2) (layer "F.Cu") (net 5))
 (segment (start 62.29 57.21) (end 62.29 67.027792) (width 0.2) (layer "F.Cu") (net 5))
 (segment (start 40.64 66.04) (end 42.45 67.85) (width 0.2) (layer "F.Cu") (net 5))
 (segment (start 55.88 40.81) (end 55.88 38.1) (width 0.2) (layer "F.Cu") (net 5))
 (segment (start 50.8 53.34) (end 51.37 52.77) (width 0.2) (layer "F.Cu") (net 5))
 (segment (start 51.37 52.77) (end 51.37 51.32) (width 0.2) (layer "F.Cu") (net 5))
 (segment (start 52.215 21.685) (end 64.865 21.685) (width 0.2) (layer "F.Cu") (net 5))
 (segment (start 51.37 23.19) (end 51.04 22.86) (width 0.2) (layer "F.Cu") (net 5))
 (segment (start 51.04 22.86) (end 52.215 21.685) (width 0.2) (layer "F.Cu") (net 5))
 (segment (start 35.2325 48.32) (end 38.2325 45.32) (width 0.2) (layer "F.Cu") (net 5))
 (segment (start 35.56 53.34) (end 35.56 48.26) (width 0.2) (layer "F.Cu") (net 5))
 (segment (start 28.45 69.32) (end 28.45 68.07) (width 0.2) (layer "F.Cu") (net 5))
 (segment (start 56.45 70.55) (end 55.88 71.12) (width 0.2) (layer "F.Cu") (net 5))
 (segment (start 35.56 48.26) (end 35.5 48.32) (width 0.2) (layer "F.Cu") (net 5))
 (segment (start 43.18 53.34) (end 46.2125 53.34) (width 0.2) (layer "F.Cu") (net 5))
 (via (at 58.42 53.34) (size 0.6) (drill 0.3) (layers "F.Cu" "B.Cu") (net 5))
 (via (at 50.8 53.34) (size 0.6) (drill 0.3) (layers "F.Cu" "B.Cu") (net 5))
 (via (at 43.18 53.34) (size 0.6) (drill 0.3) (layers "F.Cu" "B.Cu") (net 5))
 (segment (start 49.865 24.035) (end 51.04 22.86) (width 0.2) (layer "B.Cu") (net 5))
 (segment (start 39.215 24.035) (end 49.865 24.035) (width 0.2) (layer "B.Cu") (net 5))
 (segment (start 43.18 53.34) (end 50.8 53.34) (width 0.2) (layer "B.Cu") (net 5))
 (segment (start 38.04 22.86) (end 39.215 24.035) (width 0.2) (layer "B.Cu") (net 5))
 (segment (start 50.8 53.34) (end 58.42 53.34) (width 0.2) (layer "B.Cu") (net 5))
 (segment (start 59.27 51.65) (end 60.96 53.34) (width 0.2) (layer "F.Cu") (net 2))
 (segment (start 59.27 48.32) (end 59.27 51.65) (width 0.2) (layer "F.Cu") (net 2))
 (segment (start 38.1 73.66) (end 40.45 71.31) (width 0.2) (layer "F.Cu") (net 2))
 (segment (start 26.45 69.32) (end 26.45 72.17) (width 0.2) (layer "F.Cu") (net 2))
 (segment (start 53.27 35.56) (end 53.27 23.09) (width 0.2) (layer "F.Cu") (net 2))
 (segment (start 69.2575 48.32) (end 75.72 41.8575) (width 0.2) (layer "F.Cu") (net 2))
 (segment (start 63.2325 51.32) (end 66.2325 48.32) (width 0.2) (layer "F.Cu") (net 2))
 (segment (start 53.27 23.09) (end 53.04 22.86) (width 0.2) (layer "F.Cu") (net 2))
 (segment (start 75.72 41.8575) (end 75.72 35.56) (width 0.2) (layer "F.Cu") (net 2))
 (segment (start 53.34 50.267972) (end 53.34 48.26) (width 0.2) (layer "F.Cu") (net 2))
 (segment (start 61.2125 53.34) (end 63.2325 51.32) (width 0.2) (layer "F.Cu") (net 2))
 (segment (start 26.45 72.17) (end 27.94 73.66) (width 0.2) (layer "F.Cu") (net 2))
 (segment (start 60.96 53.34) (end 61.2125 53.34) (width 0.2) (layer "F.Cu") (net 2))
 (segment (start 27.94 73.66) (end 38.1 73.66) (width 0.2) (layer "F.Cu") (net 2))
 (segment (start 59.27 46.57) (end 59.27 48.32) (width 0.2) (layer "F.Cu") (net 2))
 (segment (start 53.27 51.32) (end 53.27 50.337972) (width 0.2) (layer "F.Cu") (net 2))
 (segment (start 40.45 71.31) (end 40.45 69.32) (width 0.2) (layer "F.Cu") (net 2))
 (segment (start 58.42 45.72) (end 59.27 46.57) (width 0.2) (layer "F.Cu") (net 2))
 (segment (start 55.88 45.72) (end 58.42 45.72) (width 0.2) (layer "F.Cu") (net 2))
 (segment (start 63.2325 51.32) (end 63.2325 53.0725) (width 0.2) (layer "F.Cu") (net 2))
 (segment (start 63.2325 53.0725) (end 67.37 57.21) (width 0.2) (layer "F.Cu") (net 2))
 (segment (start 53.34 48.26) (end 55.88 45.72) (width 0.2) (layer "F.Cu") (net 2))
 (segment (start 75.72 35.56) (end 53.27 35.56) (width 0.2) (layer "F.Cu") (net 2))
 (segment (start 66.2325 48.32) (end 69.2575 48.32) (width 0.2) (layer "F.Cu") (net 2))
 (segment (start 62.04 22.86) (end 53.04 22.86) (width 0.2) (layer "F.Cu") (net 2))
 (segment (start 53.27 50.337972) (end 53.34 50.267972) (width 0.2) (layer "F.Cu") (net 2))
 (segment (start 50.11 73.66) (end 54.45 69.32) (width 0.2) (layer "B.Cu") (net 2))
 (segment (start 40.04 22.86) (end 41.215 21.685) (width 0.2) (layer "B.Cu") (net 2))
 (segment (start 67.19 73.66) (end 71.53 69.32) (width 0.2) (layer "B.Cu") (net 2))
 (segment (start 51.865 21.685) (end 53.04 22.86) (width 0.2) (layer "B.Cu") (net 2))
 (segment (start 41.215 21.685) (end 51.865 21.685) (width 0.2) (layer "B.Cu") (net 2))
 (segment (start 54.45 69.32) (end 58.79 73.66) (width 0.2) (layer "B.Cu") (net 2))
 (segment (start 67.37 57.21) (end 67.37 65.16) (width 0.2) (layer "B.Cu") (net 2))
 (segment (start 40.45 69.32) (end 44.79 73.66) (width 0.2) (layer "B.Cu") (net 2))
 (segment (start 58.79 73.66) (end 67.19 73.66) (width 0.2) (layer "B.Cu") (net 2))
 (segment (start 44.79 73.66) (end 50.11 73.66) (width 0.2) (layer "B.Cu") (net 2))
 (segment (start 67.37 65.16) (end 71.53 69.32) (width 0.2) (layer "B.Cu") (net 2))
 (segment (start 61.40704 47.9425) (end 67.38366 47.9425) (width 0.1524) (layer "F.Cu") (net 8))
 (segment (start 61.40704 48.32096) (end 61.40704 47.9425) (width 0.1524) (layer "F.Cu") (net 8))
 (segment (start 67.38366 47.371) (end 67.38366 47.9425) (width 0.1524) (layer "F.Cu") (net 8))
 (segment (start 61.40704 51.3207) (end 61.40704 48.32096) (width 0.1524) (layer "F.Cu") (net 8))
 (segment (start 61.40704 47.9425) (end 61.40704 45.32122) (width 0.1524) (layer "F.Cu") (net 8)))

